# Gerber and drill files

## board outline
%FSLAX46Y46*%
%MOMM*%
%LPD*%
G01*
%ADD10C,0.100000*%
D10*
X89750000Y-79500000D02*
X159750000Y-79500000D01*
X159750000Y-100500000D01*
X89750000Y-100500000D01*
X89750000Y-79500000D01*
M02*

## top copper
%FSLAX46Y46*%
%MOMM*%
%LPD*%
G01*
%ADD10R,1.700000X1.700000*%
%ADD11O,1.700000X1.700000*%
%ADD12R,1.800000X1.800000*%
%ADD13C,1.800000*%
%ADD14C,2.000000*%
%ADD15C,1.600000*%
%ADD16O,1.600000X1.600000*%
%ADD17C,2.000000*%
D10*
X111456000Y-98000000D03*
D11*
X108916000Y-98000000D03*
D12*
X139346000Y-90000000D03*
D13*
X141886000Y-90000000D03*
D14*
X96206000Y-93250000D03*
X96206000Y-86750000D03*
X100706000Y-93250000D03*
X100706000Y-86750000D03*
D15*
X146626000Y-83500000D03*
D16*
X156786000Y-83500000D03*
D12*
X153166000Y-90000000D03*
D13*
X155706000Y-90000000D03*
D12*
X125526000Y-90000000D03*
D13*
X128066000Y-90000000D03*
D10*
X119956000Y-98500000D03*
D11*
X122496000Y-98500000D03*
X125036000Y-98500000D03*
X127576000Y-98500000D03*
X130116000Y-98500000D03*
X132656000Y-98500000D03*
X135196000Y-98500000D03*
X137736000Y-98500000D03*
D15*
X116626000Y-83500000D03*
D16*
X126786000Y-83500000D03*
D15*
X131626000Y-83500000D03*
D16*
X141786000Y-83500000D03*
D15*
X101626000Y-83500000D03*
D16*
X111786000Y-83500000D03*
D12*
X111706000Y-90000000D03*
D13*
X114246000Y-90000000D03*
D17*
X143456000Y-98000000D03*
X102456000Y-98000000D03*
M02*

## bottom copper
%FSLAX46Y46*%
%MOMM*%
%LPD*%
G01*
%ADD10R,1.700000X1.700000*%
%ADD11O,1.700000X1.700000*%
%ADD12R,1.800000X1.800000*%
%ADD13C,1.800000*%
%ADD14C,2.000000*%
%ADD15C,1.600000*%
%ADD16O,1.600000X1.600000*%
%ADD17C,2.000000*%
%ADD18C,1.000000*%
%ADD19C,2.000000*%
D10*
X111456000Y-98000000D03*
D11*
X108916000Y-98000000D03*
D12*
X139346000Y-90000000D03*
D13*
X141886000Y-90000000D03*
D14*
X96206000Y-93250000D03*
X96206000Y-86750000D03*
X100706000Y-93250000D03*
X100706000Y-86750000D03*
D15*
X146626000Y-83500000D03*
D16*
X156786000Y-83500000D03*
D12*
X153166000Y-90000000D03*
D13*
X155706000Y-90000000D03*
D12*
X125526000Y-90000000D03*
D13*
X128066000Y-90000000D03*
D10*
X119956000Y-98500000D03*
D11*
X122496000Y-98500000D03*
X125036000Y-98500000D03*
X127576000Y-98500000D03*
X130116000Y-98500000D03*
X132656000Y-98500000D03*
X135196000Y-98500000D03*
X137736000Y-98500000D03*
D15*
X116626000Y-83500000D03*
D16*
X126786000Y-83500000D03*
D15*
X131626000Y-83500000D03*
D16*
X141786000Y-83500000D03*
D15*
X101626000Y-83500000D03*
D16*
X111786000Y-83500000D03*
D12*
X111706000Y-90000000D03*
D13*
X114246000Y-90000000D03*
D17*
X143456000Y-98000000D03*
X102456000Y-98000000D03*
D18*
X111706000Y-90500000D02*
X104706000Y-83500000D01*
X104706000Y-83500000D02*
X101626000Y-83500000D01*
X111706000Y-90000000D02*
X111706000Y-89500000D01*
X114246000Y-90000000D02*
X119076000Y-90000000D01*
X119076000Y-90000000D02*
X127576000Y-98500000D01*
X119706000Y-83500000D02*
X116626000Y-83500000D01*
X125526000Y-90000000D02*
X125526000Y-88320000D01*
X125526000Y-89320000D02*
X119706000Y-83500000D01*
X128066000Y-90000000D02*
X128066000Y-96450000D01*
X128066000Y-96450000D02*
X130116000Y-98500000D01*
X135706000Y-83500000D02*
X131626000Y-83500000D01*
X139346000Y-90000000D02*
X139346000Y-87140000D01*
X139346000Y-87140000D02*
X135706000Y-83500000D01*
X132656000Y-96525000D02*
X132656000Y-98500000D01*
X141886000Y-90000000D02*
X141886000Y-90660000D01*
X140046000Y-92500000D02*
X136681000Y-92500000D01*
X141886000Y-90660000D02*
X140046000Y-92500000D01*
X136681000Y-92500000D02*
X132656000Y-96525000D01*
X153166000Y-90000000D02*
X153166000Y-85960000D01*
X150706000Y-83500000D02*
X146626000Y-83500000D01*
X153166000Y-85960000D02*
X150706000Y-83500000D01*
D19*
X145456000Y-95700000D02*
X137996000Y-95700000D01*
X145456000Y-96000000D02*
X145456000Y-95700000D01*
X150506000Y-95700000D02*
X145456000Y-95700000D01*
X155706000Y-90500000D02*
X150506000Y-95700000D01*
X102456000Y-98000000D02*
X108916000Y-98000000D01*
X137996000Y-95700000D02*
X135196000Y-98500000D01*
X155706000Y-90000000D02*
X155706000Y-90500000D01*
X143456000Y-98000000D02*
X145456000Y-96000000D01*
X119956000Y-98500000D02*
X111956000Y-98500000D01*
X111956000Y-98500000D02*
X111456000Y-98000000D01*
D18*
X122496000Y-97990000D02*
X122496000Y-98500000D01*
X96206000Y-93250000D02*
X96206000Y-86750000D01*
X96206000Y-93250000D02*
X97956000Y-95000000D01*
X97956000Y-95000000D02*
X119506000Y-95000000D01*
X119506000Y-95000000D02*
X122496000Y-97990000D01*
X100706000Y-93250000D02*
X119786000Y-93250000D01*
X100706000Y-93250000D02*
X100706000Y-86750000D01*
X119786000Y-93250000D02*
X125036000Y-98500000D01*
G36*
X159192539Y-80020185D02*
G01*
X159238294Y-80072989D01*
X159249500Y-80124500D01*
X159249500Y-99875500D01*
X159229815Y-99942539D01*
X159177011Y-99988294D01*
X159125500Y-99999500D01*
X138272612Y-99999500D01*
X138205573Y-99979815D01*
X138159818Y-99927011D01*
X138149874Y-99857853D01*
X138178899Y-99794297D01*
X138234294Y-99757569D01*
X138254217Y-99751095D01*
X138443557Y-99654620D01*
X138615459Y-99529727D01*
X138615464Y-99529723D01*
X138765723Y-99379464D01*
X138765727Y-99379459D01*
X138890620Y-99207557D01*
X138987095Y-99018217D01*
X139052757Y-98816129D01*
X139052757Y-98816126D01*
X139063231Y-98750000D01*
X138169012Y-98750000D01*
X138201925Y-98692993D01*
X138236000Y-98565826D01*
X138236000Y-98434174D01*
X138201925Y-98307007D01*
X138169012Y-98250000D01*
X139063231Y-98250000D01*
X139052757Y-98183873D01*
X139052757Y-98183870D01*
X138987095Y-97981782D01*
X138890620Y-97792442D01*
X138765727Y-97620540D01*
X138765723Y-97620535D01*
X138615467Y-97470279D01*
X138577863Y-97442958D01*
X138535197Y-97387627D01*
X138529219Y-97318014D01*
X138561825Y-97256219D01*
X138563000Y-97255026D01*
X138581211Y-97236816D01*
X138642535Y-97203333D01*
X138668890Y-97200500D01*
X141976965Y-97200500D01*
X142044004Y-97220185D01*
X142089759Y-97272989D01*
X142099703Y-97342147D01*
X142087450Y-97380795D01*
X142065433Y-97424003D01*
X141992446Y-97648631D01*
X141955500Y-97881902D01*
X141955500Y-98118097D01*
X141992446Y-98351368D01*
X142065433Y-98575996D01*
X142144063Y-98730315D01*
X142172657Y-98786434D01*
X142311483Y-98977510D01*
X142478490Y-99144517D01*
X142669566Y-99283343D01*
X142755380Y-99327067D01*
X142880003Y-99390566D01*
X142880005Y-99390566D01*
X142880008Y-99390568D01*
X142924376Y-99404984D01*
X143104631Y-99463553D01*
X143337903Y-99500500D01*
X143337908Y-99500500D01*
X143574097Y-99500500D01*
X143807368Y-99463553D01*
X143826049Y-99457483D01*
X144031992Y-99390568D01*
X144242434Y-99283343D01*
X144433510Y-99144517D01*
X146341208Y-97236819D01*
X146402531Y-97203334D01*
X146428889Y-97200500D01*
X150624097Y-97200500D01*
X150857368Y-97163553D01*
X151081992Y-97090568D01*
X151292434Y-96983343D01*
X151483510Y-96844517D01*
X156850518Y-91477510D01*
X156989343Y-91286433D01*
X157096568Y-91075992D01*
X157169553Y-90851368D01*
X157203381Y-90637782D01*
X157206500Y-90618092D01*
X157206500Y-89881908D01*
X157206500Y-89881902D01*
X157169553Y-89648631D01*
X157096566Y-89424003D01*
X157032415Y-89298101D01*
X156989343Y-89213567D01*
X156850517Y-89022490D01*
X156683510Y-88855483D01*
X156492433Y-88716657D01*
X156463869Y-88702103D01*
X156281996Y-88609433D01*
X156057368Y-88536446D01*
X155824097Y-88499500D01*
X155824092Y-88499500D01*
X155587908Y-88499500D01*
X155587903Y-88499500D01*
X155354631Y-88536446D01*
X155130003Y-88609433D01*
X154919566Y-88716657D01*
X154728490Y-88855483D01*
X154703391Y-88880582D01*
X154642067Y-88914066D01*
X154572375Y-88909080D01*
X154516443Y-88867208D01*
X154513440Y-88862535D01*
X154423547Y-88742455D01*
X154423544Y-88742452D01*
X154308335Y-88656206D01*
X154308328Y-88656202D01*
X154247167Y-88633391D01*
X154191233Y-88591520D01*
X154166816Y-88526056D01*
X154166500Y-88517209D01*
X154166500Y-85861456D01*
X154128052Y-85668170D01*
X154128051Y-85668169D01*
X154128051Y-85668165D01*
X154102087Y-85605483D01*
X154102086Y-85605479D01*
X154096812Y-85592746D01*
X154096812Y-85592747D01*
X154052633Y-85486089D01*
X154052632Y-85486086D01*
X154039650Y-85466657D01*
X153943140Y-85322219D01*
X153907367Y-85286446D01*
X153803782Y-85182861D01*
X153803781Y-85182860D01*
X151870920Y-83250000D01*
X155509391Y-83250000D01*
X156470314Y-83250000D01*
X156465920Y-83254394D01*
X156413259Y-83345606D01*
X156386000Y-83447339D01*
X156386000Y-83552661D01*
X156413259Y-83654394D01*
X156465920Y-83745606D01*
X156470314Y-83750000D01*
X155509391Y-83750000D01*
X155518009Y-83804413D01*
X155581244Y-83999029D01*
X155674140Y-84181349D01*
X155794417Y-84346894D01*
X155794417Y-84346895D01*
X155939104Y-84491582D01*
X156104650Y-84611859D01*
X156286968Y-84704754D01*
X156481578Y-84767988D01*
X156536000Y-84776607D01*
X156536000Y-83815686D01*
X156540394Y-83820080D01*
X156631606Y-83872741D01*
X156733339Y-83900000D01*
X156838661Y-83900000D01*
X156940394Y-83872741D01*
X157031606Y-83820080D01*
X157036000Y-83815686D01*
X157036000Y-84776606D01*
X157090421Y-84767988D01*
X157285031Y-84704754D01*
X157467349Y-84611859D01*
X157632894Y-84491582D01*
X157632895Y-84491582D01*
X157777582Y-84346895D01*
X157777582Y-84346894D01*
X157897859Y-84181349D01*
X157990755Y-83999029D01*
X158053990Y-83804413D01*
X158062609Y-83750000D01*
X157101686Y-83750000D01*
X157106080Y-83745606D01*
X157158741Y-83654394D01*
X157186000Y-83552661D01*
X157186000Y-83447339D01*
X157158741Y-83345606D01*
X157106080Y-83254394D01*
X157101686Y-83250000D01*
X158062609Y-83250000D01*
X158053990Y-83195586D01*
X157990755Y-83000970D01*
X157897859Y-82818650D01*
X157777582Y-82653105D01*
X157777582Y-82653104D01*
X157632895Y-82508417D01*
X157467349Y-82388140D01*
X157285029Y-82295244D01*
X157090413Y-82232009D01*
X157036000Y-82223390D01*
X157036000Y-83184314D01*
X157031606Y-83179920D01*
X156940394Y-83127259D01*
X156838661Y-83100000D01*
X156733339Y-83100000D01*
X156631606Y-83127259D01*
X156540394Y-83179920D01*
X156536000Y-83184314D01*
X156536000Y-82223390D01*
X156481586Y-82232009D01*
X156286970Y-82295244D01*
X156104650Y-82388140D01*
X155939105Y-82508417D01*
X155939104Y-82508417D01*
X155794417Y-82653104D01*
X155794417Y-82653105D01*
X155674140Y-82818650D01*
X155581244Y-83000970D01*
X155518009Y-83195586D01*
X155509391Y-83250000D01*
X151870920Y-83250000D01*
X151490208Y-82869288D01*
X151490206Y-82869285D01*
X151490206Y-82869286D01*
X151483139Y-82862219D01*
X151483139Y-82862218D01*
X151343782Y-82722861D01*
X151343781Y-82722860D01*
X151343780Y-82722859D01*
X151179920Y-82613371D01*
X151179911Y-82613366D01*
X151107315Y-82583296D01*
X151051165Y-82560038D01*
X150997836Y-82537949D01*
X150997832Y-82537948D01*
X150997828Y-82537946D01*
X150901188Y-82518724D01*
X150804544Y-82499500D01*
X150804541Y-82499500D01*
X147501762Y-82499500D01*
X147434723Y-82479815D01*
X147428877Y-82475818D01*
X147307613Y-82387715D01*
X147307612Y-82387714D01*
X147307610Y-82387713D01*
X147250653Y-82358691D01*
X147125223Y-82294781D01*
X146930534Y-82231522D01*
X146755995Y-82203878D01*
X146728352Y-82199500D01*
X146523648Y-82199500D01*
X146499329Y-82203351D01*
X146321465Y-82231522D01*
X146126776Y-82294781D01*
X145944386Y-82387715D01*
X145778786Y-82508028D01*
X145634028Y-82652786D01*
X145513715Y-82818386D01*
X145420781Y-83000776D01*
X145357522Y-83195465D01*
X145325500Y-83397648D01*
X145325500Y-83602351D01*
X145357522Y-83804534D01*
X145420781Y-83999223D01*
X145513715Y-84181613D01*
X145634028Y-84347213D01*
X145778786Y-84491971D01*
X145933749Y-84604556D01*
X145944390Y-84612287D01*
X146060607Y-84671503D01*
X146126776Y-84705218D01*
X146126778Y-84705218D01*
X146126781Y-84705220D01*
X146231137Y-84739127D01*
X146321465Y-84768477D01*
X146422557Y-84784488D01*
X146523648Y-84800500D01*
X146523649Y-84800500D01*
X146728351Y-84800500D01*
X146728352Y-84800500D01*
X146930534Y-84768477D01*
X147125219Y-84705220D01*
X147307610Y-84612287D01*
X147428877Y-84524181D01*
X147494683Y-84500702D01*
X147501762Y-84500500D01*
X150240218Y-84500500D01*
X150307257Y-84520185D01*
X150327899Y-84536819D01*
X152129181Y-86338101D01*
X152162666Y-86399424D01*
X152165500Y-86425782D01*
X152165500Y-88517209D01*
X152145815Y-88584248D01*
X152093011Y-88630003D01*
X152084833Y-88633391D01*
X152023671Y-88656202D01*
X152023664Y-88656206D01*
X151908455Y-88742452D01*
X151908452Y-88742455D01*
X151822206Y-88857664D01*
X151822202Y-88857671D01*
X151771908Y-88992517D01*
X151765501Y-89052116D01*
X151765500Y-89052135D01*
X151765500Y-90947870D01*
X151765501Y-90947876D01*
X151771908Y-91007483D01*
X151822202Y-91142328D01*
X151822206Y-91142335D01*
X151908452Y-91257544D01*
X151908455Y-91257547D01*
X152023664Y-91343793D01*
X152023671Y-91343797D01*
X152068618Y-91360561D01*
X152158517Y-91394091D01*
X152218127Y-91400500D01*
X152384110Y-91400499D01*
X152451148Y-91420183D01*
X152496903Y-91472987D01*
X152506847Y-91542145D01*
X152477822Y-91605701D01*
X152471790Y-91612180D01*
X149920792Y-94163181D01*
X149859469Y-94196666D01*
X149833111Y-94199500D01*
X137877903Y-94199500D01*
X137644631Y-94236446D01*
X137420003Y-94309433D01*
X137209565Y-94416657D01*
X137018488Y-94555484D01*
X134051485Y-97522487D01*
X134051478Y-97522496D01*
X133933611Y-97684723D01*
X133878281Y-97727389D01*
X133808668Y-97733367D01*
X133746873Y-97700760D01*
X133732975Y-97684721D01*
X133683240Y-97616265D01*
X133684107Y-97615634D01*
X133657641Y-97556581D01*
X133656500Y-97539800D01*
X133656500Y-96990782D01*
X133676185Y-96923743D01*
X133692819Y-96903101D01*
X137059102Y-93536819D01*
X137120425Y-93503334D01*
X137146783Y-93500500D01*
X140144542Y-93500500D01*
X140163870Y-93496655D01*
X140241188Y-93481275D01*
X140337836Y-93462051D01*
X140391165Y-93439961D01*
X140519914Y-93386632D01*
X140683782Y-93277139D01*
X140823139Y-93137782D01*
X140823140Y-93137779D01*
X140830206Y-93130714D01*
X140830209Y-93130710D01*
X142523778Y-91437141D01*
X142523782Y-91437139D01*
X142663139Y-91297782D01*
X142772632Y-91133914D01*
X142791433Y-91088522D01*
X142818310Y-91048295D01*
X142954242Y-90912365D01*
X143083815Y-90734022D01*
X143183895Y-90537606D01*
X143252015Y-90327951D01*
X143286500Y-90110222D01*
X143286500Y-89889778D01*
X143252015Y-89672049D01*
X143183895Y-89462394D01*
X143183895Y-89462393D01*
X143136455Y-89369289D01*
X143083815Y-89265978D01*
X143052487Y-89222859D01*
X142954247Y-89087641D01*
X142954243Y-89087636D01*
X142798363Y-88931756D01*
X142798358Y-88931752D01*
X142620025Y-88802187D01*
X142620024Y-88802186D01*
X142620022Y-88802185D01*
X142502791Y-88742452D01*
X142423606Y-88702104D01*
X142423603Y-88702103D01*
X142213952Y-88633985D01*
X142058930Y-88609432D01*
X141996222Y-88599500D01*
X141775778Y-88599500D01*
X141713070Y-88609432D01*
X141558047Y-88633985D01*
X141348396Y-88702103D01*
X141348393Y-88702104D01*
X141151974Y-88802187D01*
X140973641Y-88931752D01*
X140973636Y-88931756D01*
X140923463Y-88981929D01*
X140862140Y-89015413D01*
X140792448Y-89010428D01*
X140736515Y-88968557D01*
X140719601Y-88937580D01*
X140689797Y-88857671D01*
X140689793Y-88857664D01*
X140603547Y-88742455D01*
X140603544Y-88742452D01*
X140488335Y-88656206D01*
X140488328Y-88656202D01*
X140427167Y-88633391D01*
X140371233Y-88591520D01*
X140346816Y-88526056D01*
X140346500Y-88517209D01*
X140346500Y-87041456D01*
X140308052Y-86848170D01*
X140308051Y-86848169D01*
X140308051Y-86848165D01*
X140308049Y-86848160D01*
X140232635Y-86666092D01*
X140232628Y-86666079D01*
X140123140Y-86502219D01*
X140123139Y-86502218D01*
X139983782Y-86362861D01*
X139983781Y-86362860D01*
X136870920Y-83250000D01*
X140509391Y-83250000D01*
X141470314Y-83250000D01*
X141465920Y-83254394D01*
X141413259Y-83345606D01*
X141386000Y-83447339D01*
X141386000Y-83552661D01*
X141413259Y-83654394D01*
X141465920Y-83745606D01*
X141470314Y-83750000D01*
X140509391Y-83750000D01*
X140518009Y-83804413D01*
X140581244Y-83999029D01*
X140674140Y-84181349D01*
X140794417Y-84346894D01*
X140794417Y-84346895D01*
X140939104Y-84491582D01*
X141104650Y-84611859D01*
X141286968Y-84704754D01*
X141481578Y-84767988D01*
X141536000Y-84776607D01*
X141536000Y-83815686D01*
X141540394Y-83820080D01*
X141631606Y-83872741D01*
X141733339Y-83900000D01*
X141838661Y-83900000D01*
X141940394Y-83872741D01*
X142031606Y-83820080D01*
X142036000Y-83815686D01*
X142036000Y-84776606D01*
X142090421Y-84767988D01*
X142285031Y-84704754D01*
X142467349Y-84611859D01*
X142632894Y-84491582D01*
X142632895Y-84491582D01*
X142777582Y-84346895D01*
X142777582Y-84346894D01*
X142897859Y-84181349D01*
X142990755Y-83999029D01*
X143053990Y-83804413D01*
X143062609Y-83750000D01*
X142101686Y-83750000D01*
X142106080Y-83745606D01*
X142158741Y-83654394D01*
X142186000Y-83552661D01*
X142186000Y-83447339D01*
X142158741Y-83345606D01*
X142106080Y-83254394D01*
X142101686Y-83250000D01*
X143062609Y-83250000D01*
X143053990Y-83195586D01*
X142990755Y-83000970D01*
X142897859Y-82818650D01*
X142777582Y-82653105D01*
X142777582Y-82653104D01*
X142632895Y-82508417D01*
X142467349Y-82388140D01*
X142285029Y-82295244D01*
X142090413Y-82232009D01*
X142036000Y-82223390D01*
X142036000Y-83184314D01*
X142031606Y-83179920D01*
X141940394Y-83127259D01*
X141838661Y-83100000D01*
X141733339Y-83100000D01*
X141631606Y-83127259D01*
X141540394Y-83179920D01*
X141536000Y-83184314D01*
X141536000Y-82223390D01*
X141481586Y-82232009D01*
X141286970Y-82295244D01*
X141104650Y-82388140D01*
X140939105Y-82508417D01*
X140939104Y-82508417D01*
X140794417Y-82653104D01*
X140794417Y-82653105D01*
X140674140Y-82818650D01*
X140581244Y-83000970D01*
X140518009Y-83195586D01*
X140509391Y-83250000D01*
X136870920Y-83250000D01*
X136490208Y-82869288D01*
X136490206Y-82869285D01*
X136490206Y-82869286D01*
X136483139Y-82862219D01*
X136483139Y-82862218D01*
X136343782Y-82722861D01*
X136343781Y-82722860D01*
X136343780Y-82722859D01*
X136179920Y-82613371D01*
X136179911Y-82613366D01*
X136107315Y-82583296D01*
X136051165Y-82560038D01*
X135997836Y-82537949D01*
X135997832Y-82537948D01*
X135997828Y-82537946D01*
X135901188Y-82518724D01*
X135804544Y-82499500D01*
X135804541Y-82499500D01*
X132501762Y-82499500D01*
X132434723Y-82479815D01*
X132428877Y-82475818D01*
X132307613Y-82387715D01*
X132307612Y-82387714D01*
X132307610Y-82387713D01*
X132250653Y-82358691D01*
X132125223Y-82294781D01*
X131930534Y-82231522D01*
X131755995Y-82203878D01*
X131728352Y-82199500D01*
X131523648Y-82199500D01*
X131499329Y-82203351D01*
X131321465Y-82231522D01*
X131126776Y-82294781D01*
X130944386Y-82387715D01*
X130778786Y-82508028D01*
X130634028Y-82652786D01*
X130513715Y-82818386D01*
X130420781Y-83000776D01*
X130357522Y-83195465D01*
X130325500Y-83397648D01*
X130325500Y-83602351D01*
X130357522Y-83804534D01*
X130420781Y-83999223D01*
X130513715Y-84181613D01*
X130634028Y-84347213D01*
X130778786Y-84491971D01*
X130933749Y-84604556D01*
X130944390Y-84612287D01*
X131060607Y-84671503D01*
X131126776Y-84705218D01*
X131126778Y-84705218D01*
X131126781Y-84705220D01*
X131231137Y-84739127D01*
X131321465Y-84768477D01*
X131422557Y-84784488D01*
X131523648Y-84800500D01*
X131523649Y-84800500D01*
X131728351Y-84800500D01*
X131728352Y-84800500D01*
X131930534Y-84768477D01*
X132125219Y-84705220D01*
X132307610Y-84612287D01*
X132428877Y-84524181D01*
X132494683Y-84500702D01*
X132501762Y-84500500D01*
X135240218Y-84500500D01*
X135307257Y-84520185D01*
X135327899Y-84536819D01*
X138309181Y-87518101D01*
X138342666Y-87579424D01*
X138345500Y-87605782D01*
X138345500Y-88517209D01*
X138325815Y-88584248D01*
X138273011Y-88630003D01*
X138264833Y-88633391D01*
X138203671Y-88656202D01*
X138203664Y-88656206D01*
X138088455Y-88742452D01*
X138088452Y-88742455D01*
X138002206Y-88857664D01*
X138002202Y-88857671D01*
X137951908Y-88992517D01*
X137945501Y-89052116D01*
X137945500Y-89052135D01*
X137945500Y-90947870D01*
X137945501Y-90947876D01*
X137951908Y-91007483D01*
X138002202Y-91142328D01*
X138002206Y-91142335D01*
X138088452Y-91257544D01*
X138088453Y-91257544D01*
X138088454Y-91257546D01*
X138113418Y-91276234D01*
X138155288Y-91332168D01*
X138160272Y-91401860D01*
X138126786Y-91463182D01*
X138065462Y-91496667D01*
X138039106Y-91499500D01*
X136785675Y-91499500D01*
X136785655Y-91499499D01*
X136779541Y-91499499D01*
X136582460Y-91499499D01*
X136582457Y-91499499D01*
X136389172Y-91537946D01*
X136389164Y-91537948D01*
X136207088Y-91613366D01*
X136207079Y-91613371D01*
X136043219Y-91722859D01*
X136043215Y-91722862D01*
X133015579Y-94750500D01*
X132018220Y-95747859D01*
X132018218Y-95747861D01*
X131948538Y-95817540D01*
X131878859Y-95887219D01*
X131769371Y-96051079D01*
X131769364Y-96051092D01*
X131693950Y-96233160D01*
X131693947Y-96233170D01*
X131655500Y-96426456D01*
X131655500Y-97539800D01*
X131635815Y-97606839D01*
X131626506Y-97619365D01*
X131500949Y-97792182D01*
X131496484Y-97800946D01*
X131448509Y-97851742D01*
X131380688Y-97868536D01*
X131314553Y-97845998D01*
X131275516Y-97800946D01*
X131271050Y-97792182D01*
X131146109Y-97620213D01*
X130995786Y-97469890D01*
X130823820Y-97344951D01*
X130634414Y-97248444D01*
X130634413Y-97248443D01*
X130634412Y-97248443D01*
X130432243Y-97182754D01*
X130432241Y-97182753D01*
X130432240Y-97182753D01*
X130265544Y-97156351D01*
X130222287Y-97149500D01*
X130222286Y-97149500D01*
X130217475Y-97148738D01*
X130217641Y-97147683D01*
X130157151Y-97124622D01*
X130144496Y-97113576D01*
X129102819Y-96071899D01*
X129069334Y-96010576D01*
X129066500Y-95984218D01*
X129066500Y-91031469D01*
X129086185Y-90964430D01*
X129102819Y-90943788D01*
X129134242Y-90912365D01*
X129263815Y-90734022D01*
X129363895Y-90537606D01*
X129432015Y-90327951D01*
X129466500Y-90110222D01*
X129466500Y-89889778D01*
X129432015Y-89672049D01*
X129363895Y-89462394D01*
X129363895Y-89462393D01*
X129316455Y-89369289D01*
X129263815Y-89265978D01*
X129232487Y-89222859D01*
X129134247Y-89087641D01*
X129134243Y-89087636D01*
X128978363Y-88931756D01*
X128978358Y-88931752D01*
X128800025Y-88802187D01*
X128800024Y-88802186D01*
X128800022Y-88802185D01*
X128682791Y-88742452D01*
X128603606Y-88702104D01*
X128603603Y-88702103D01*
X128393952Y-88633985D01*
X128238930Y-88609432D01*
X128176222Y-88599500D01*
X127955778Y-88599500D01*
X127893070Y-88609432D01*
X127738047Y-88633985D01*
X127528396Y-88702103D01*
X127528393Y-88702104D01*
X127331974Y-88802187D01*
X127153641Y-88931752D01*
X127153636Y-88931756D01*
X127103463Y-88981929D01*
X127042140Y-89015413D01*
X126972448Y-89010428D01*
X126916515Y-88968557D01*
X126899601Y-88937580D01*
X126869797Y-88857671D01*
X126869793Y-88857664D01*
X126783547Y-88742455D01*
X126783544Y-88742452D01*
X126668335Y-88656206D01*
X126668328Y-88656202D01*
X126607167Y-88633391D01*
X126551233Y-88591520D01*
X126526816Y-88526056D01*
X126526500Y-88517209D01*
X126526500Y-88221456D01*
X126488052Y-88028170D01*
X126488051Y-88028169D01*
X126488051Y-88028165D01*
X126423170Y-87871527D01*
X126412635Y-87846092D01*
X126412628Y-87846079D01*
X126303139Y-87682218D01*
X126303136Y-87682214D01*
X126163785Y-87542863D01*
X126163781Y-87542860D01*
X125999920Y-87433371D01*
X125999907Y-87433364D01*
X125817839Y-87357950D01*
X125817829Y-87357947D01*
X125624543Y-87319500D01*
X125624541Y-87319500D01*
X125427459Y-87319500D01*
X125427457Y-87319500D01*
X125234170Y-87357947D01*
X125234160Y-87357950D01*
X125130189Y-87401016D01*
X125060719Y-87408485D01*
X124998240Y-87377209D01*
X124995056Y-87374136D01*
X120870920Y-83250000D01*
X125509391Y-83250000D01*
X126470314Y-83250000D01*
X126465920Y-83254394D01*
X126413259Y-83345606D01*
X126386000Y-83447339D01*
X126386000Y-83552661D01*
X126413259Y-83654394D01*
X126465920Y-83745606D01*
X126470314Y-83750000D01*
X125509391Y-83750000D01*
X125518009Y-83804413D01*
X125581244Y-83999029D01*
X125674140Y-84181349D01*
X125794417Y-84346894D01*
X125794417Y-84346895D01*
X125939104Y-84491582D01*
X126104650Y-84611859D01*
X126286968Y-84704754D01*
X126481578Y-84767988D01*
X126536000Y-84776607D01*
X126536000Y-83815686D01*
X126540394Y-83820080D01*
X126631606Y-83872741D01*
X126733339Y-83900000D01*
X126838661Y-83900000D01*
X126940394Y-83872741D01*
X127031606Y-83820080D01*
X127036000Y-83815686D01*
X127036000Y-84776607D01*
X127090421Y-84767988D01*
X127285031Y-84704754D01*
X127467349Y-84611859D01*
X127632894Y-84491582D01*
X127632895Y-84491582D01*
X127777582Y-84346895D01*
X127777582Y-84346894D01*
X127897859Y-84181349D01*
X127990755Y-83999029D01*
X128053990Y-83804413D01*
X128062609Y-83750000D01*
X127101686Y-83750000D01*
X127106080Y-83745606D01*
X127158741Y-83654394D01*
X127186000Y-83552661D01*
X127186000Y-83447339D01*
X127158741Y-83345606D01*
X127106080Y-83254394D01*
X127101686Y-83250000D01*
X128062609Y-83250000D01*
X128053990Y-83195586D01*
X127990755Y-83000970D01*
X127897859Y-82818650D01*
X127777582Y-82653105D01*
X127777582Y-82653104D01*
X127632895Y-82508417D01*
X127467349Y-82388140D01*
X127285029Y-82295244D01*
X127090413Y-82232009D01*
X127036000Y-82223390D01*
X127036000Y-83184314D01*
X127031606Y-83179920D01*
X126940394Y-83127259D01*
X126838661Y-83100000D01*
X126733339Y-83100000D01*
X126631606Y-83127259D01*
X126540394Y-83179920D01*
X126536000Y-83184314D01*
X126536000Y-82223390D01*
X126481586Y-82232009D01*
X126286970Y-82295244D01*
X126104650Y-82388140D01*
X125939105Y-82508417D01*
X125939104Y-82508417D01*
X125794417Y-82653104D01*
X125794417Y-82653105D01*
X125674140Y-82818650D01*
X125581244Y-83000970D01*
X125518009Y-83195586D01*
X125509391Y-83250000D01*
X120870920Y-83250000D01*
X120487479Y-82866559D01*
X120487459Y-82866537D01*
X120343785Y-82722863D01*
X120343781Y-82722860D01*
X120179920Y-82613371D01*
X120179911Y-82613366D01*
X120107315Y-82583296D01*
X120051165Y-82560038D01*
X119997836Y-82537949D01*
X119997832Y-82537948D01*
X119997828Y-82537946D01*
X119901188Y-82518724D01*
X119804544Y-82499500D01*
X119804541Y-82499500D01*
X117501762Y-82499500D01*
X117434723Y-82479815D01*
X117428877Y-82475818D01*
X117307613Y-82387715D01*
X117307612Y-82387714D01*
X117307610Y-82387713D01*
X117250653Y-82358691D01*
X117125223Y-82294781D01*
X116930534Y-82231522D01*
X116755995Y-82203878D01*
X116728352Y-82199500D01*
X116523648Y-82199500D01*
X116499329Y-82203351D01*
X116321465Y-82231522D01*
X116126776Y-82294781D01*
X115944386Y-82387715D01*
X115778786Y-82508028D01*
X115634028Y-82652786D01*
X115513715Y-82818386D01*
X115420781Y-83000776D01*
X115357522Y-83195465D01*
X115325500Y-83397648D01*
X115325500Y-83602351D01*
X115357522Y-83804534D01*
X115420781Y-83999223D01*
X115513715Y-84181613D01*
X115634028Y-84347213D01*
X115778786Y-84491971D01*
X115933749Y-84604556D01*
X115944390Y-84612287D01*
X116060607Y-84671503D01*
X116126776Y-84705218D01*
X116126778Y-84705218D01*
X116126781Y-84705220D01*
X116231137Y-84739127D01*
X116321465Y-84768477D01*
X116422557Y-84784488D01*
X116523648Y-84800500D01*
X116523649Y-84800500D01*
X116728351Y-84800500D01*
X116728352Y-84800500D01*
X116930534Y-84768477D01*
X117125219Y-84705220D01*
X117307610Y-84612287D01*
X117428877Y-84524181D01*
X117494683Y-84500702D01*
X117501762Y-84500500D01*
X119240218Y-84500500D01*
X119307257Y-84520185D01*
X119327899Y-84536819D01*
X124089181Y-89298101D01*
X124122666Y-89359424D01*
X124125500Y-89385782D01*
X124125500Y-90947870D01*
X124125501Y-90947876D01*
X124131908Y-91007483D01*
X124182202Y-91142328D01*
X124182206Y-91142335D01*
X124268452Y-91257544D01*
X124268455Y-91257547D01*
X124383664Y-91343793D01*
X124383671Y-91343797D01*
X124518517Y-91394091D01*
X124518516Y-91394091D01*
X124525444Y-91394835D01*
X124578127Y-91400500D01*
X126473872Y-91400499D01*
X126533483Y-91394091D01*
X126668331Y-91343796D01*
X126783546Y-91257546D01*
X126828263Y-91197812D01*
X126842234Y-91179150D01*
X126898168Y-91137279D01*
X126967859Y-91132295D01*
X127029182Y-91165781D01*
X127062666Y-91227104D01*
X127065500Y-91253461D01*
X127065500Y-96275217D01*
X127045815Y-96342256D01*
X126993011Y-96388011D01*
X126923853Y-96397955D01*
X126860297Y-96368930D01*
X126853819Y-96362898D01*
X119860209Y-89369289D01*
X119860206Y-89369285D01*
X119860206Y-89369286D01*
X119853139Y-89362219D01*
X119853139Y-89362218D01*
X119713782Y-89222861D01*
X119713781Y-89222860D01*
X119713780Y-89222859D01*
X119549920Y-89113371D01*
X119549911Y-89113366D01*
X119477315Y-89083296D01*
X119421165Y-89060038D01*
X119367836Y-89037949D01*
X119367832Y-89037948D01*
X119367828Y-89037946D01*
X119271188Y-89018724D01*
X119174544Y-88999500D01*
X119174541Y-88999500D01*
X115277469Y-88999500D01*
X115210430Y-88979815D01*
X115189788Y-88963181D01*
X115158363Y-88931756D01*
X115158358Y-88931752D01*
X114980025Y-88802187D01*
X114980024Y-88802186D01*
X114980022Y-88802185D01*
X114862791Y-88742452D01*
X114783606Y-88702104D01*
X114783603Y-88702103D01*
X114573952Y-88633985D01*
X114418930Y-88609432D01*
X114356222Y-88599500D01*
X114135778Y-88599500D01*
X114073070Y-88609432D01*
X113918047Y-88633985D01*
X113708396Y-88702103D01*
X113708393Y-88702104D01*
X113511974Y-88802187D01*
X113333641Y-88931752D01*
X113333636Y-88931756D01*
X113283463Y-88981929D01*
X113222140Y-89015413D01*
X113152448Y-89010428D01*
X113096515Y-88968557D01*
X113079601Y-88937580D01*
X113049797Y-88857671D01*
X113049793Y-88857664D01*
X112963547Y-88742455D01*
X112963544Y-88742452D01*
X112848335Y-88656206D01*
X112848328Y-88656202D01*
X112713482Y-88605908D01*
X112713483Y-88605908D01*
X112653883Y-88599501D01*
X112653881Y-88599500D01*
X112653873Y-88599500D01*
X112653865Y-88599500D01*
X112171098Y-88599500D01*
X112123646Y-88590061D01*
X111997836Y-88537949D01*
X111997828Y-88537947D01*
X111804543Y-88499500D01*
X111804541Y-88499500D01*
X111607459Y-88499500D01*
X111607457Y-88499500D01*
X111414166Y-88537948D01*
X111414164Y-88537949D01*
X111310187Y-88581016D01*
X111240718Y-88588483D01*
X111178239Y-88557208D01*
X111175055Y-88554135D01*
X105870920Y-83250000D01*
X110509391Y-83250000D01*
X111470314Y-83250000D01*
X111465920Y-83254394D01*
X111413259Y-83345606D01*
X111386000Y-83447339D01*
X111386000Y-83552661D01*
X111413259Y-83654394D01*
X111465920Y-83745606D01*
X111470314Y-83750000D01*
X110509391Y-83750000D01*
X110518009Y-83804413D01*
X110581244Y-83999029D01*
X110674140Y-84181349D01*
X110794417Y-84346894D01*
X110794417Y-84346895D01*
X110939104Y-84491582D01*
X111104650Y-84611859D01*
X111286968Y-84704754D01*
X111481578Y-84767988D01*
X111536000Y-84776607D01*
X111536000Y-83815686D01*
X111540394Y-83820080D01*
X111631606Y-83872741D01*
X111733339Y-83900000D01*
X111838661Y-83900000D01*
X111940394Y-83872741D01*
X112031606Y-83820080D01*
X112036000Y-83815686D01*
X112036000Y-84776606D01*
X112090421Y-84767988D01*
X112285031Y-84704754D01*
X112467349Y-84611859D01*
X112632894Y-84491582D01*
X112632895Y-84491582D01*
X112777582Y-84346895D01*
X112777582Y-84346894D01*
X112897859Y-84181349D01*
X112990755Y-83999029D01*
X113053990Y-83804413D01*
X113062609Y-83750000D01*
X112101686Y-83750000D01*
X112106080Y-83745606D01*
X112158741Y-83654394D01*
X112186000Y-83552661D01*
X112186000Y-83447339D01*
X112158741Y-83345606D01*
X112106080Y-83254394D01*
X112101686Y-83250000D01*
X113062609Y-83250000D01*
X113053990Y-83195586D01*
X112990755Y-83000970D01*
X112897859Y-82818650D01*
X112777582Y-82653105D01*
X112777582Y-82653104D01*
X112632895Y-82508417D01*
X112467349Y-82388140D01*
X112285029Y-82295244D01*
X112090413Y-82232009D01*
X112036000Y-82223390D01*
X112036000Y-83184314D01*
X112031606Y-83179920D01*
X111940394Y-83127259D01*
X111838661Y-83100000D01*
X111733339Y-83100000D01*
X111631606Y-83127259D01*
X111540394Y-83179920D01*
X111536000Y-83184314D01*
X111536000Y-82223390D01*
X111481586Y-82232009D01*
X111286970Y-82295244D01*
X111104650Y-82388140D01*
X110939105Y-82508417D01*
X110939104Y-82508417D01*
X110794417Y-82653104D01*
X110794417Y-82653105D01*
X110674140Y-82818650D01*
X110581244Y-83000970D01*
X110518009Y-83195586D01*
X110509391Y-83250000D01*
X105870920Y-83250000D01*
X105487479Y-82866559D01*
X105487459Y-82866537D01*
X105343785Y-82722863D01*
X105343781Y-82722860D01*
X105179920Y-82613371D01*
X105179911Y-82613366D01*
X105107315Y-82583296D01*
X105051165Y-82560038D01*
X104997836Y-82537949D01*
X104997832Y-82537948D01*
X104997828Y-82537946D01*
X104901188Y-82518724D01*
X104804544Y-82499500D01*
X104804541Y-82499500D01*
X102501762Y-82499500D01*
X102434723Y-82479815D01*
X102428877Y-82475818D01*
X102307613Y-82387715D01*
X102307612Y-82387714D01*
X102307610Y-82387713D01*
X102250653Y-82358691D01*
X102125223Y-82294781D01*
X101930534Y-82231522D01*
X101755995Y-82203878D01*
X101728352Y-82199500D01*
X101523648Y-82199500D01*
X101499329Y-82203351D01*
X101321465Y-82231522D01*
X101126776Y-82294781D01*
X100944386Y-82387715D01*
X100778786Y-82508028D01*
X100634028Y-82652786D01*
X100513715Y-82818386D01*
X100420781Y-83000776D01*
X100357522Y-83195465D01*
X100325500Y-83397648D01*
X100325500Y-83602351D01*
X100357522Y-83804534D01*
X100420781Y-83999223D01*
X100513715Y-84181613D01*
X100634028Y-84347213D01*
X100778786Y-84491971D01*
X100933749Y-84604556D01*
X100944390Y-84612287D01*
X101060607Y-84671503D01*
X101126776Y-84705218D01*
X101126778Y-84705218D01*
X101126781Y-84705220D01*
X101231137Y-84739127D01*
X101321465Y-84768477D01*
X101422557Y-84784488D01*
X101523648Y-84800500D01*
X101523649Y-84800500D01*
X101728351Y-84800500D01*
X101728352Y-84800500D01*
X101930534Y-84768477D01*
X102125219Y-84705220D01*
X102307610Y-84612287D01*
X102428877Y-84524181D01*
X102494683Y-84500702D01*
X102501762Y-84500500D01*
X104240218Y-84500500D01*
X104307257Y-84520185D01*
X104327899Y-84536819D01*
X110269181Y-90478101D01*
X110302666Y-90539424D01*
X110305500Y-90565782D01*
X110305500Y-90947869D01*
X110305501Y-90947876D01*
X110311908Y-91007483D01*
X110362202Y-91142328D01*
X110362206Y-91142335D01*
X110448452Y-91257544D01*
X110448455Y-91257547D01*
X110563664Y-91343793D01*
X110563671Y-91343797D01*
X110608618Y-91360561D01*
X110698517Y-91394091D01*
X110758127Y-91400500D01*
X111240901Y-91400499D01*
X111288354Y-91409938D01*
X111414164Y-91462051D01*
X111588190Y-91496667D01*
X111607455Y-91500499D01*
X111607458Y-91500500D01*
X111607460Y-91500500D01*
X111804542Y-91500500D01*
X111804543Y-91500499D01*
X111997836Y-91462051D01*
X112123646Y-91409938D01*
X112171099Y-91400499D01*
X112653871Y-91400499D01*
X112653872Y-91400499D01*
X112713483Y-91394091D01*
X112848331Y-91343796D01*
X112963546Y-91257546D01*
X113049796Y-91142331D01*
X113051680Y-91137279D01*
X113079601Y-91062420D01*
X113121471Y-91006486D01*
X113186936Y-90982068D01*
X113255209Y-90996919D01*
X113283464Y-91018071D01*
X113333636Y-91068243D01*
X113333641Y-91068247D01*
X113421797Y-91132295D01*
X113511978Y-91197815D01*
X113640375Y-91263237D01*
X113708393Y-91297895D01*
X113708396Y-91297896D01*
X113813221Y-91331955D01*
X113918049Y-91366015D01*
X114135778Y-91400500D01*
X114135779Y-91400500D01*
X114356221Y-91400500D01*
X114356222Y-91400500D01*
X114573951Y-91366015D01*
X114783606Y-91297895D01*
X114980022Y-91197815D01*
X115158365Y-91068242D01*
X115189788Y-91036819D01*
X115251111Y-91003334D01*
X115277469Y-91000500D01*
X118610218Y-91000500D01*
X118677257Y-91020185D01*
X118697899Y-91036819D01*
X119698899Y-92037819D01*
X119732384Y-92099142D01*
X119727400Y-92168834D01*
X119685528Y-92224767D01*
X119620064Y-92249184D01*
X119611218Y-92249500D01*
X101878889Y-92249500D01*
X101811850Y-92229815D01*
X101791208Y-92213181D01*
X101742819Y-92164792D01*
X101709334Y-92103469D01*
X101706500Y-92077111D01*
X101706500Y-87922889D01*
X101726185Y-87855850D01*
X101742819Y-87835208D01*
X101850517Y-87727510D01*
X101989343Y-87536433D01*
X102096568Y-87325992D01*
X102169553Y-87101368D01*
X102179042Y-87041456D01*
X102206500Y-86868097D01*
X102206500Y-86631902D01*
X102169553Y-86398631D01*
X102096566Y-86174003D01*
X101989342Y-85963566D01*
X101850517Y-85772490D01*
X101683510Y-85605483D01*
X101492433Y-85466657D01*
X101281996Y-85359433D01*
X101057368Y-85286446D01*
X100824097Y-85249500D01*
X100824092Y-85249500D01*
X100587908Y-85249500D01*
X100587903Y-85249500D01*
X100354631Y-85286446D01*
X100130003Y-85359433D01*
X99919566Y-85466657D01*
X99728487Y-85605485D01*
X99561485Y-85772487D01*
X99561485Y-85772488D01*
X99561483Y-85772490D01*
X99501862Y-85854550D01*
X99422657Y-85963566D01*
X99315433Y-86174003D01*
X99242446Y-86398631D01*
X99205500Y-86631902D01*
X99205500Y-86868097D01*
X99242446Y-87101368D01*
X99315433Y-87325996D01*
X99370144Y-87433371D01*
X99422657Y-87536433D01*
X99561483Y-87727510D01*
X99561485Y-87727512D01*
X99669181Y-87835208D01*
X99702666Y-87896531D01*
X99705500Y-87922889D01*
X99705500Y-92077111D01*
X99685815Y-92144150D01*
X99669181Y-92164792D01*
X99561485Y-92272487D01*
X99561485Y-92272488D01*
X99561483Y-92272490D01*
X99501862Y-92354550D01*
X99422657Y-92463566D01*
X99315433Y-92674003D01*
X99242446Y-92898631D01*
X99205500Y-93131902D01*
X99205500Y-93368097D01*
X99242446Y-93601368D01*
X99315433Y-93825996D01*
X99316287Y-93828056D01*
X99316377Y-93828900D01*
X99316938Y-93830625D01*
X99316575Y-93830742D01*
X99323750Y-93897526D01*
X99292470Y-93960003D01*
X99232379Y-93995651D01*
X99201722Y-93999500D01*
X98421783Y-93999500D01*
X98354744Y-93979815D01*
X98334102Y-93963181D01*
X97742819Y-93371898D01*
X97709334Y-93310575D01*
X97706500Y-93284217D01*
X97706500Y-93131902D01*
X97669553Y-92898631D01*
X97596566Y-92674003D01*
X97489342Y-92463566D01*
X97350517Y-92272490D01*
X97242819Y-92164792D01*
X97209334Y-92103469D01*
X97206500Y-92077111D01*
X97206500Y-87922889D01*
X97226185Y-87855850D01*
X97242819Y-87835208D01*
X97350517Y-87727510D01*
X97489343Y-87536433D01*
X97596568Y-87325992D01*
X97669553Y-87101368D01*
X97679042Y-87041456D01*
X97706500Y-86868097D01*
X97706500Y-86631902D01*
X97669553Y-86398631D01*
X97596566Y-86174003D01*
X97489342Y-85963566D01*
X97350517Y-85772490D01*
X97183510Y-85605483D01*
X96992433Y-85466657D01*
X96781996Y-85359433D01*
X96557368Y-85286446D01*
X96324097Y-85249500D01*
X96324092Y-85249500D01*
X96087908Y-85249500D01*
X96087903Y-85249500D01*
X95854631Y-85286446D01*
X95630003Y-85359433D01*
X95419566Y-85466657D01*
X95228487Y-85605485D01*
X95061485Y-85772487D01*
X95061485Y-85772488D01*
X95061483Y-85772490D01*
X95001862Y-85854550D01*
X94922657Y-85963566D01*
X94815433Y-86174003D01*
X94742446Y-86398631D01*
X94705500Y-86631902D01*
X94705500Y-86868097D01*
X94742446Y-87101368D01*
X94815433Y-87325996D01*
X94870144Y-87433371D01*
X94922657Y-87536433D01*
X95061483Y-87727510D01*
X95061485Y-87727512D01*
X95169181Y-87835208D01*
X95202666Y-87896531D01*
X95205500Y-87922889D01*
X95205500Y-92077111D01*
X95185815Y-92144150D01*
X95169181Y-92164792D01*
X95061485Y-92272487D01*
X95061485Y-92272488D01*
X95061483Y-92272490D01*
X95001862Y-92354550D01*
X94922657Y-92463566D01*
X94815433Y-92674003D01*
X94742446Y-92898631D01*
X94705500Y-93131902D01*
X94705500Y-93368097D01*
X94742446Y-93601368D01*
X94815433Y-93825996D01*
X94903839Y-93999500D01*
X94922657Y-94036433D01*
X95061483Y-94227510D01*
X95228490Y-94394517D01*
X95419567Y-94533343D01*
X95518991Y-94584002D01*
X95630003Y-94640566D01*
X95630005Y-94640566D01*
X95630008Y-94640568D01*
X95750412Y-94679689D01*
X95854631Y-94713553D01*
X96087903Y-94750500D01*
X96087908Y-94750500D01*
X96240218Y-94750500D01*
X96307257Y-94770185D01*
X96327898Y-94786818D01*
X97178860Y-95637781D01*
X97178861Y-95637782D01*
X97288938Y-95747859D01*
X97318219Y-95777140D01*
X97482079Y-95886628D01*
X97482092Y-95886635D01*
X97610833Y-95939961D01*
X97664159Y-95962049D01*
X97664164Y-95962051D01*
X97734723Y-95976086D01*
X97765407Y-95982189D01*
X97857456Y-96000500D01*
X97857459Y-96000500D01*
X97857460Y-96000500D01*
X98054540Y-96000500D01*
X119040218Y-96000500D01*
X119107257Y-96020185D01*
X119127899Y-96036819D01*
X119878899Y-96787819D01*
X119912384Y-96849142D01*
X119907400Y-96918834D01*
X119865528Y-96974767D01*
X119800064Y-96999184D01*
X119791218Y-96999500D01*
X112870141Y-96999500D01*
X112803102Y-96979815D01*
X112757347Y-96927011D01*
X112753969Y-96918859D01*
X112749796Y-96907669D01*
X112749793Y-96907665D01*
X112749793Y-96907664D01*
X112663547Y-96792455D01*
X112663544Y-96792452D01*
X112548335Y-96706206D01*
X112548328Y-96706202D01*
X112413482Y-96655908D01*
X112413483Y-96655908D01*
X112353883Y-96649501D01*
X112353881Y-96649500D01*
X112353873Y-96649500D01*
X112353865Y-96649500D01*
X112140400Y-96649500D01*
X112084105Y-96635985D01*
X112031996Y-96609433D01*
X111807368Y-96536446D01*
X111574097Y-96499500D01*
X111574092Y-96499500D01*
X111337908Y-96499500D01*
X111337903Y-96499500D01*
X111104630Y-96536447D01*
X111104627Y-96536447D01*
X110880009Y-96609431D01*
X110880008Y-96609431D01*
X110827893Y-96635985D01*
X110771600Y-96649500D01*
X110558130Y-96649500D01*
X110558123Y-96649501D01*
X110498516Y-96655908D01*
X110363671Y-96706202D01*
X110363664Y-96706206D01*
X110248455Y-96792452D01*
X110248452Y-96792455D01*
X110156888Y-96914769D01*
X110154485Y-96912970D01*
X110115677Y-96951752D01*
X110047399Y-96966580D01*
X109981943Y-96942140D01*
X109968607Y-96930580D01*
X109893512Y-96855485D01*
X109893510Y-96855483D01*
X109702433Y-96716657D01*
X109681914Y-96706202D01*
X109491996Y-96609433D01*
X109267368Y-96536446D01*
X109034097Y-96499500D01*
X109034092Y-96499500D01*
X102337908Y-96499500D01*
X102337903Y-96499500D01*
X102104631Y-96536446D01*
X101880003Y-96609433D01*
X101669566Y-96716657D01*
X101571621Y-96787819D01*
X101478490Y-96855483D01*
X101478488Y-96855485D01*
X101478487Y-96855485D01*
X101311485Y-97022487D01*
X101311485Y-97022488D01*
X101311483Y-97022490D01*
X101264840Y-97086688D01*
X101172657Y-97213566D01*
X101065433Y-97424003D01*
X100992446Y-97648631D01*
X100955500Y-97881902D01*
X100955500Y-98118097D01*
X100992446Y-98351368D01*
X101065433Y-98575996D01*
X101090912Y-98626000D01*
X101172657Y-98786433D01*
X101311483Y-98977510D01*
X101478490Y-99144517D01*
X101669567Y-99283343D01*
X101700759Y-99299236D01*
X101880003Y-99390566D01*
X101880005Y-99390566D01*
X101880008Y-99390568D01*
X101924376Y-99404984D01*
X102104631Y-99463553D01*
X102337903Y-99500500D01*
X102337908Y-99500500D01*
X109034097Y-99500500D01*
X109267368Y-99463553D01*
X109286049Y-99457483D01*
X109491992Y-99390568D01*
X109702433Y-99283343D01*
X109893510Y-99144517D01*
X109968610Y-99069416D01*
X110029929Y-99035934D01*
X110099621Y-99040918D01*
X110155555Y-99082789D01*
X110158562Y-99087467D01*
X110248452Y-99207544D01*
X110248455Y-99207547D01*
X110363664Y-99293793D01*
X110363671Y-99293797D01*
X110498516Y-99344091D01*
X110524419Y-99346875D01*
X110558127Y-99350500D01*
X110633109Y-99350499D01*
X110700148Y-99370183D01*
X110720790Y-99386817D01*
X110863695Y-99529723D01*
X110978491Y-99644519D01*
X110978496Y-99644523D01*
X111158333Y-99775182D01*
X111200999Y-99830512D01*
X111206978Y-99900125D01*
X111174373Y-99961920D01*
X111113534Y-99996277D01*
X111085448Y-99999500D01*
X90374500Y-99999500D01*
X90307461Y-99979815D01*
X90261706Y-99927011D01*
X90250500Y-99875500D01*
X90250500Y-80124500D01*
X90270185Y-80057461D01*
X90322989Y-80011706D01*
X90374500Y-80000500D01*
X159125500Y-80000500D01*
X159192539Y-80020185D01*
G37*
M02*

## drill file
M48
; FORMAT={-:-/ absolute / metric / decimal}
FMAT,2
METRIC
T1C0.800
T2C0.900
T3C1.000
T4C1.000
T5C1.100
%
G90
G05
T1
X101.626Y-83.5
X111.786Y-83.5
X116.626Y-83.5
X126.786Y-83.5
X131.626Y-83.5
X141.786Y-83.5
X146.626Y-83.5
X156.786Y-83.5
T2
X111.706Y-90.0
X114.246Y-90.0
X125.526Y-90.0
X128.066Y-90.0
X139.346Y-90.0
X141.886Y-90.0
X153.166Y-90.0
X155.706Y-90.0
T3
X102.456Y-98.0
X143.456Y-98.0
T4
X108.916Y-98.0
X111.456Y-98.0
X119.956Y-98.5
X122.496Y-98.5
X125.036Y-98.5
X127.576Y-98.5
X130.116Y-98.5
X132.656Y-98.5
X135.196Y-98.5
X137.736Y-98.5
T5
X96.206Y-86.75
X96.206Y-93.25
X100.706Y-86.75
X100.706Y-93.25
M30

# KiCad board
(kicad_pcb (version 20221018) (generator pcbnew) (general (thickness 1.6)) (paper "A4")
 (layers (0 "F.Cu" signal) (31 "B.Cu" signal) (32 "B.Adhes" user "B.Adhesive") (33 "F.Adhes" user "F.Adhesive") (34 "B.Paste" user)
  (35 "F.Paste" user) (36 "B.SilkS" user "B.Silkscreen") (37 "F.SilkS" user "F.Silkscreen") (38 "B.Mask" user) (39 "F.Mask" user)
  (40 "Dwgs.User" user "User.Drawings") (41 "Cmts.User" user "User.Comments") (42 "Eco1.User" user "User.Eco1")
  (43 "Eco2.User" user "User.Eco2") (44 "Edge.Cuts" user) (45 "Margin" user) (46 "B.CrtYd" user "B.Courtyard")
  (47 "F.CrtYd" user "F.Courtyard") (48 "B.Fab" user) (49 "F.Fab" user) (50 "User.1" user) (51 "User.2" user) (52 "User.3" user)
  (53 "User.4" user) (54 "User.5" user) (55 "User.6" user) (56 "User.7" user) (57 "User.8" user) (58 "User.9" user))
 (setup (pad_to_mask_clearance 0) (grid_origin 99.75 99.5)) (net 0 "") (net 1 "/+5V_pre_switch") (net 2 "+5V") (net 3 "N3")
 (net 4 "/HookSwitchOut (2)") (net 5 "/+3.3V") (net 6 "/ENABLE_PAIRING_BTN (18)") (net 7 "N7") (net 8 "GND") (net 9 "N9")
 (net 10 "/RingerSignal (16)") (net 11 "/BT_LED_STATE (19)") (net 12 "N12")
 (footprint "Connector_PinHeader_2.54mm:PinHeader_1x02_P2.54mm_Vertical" (layer "F.Cu") (at 111.456 98 -90)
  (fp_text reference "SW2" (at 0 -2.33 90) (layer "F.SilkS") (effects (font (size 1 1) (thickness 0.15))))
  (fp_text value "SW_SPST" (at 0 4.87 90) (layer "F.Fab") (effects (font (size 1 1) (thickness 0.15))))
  (pad "1" thru_hole rect (at 0 0 270) (size 1.7 1.7) (drill 1) (layers "*.Cu" "*.Mask") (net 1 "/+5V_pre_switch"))
  (pad "2" thru_hole oval (at 0 2.54 270) (size 1.7 1.7) (drill 1) (layers "*.Cu" "*.Mask") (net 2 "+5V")))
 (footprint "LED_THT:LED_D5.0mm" (layer "F.Cu") (at 139.346 90)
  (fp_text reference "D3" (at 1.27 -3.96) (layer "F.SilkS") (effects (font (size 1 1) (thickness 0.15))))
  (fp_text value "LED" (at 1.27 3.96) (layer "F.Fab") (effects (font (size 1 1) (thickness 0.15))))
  (pad "1" thru_hole rect (at 0 0) (size 1.8 1.8) (drill 0.9) (layers "*.Cu" "*.Mask") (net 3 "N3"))
  (pad "2" thru_hole circle (at 2.54 0) (size 1.8 1.8) (drill 0.9) (layers "*.Cu" "*.Mask") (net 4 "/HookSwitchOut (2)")))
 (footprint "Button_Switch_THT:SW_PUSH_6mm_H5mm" (layer "F.Cu") (at 96.206 93.25 90)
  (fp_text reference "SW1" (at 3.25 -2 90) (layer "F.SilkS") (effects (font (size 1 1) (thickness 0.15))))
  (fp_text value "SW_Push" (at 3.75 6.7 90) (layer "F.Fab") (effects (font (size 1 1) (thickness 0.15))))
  (pad "1" thru_hole circle (at 0 0 180) (size 2 2) (drill 1.1) (layers "*.Cu" "*.Mask") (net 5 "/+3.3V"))
  (pad "1" thru_hole circle (at 6.5 0 180) (size 2 2) (drill 1.1) (layers "*.Cu" "*.Mask") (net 5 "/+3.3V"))
  (pad "2" thru_hole circle (at 0 4.5 180) (size 2 2) (drill 1.1) (layers "*.Cu" "*.Mask") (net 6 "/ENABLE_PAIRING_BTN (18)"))
  (pad "2" thru_hole circle (at 6.5 4.5 180) (size 2 2) (drill 1.1) (layers "*.Cu" "*.Mask") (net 6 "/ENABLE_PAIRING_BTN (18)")))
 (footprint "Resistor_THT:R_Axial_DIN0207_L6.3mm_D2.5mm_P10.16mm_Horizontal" (layer "F.Cu") (at 146.626 83.5)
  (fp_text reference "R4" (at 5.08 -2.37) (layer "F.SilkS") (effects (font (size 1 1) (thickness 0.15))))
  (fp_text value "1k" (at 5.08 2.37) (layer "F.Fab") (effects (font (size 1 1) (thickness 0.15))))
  (pad "1" thru_hole circle (at 0 0) (size 1.6 1.6) (drill 0.8) (layers "*.Cu" "*.Mask") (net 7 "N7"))
  (pad "2" thru_hole oval (at 10.16 0) (size 1.6 1.6) (drill 0.8) (layers "*.Cu" "*.Mask") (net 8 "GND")))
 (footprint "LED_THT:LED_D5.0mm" (layer "F.Cu") (at 153.166 90)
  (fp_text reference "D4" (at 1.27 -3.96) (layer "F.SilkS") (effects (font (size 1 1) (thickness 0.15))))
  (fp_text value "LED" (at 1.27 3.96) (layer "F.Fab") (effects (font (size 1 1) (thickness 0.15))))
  (pad "1" thru_hole rect (at 0 0) (size 1.8 1.8) (drill 0.9) (layers "*.Cu" "*.Mask") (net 7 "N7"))
  (pad "2" thru_hole circle (at 2.54 0) (size 1.8 1.8) (drill 0.9) (layers "*.Cu" "*.Mask") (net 2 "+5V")))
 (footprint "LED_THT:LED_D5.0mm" (layer "F.Cu") (at 125.526 90)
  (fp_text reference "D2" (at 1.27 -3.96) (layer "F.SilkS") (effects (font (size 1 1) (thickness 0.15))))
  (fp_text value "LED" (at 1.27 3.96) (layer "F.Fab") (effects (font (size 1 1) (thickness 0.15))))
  (pad "1" thru_hole rect (at 0 0) (size 1.8 1.8) (drill 0.9) (layers "*.Cu" "*.Mask") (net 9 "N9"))
  (pad "2" thru_hole circle (at 2.54 0) (size 1.8 1.8) (drill 0.9) (layers "*.Cu" "*.Mask") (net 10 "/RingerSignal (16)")))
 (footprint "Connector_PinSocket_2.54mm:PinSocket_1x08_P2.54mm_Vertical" (layer "F.Cu") (at 119.956 98.5 90)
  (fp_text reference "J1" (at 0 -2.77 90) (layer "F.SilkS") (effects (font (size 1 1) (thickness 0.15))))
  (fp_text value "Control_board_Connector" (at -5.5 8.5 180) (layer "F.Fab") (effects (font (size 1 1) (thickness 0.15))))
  (pad "1" thru_hole rect (at 0 0 90) (size 1.7 1.7) (drill 1) (layers "*.Cu" "*.Mask") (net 1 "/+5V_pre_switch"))
  (pad "2" thru_hole oval (at 0 2.54 90) (size 1.7 1.7) (drill 1) (layers "*.Cu" "*.Mask") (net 5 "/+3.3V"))
  (pad "3" thru_hole oval (at 0 5.08 90) (size 1.7 1.7) (drill 1) (layers "*.Cu" "*.Mask") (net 6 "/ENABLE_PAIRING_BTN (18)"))
  (pad "4" thru_hole oval (at 0 7.62 90) (size 1.7 1.7) (drill 1) (layers "*.Cu" "*.Mask") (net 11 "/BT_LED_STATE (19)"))
  (pad "5" thru_hole oval (at 0 10.16 90) (size 1.7 1.7) (drill 1) (layers "*.Cu" "*.Mask") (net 10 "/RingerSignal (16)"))
  (pad "6" thru_hole oval (at 0 12.7 90) (size 1.7 1.7) (drill 1) (layers "*.Cu" "*.Mask") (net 4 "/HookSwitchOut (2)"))
  (pad "7" thru_hole oval (at 0 15.24 90) (size 1.7 1.7) (drill 1) (layers "*.Cu" "*.Mask") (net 2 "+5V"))
  (pad "8" thru_hole oval (at 0 17.78 90) (size 1.7 1.7) (drill 1) (layers "*.Cu" "*.Mask") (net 8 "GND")))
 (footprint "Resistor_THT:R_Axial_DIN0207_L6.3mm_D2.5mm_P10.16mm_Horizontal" (layer "F.Cu") (at 116.626 83.5)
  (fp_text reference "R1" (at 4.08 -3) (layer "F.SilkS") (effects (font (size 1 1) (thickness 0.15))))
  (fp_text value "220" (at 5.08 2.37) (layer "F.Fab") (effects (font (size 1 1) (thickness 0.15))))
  (pad "1" thru_hole circle (at 0 0) (size 1.6 1.6) (drill 0.8) (layers "*.Cu" "*.Mask") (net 9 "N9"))
  (pad "2" thru_hole oval (at 10.16 0) (size 1.6 1.6) (drill 0.8) (layers "*.Cu" "*.Mask") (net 8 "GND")))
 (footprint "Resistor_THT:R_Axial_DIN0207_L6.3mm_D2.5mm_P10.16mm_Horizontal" (layer "F.Cu") (at 131.626 83.5)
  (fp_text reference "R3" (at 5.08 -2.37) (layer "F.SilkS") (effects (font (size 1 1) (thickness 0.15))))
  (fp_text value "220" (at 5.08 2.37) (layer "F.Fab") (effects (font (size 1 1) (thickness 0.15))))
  (pad "1" thru_hole circle (at 0 0) (size 1.6 1.6) (drill 0.8) (layers "*.Cu" "*.Mask") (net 3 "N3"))
  (pad "2" thru_hole oval (at 10.16 0) (size 1.6 1.6) (drill 0.8) (layers "*.Cu" "*.Mask") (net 8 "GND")))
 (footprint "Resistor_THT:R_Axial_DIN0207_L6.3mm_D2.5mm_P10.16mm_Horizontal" (layer "F.Cu") (at 101.626 83.5)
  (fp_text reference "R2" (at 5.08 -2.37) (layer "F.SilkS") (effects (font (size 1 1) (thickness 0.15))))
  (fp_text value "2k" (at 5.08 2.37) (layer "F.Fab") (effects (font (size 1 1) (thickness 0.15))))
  (pad "1" thru_hole circle (at 0 0) (size 1.6 1.6) (drill 0.8) (layers "*.Cu" "*.Mask") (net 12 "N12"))
  (pad "2" thru_hole oval (at 10.16 0) (size 1.6 1.6) (drill 0.8) (layers "*.Cu" "*.Mask") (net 8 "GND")))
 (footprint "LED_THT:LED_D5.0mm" (layer "F.Cu") (at 111.706 90)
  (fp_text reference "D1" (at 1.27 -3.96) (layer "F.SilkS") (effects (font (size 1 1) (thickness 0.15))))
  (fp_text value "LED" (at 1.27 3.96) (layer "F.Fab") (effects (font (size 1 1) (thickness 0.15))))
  (pad "1" thru_hole rect (at 0 0) (size 1.8 1.8) (drill 0.9) (layers "*.Cu" "*.Mask") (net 12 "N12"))
  (pad "2" thru_hole circle (at 2.54 0) (size 1.8 1.8) (drill 0.9) (layers "*.Cu" "*.Mask") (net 11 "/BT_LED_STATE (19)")))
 (gr_rect (start 89.75 79.5) (end 159.75 100.5) (stroke (width 0.1) (type default)) (fill none) (layer "Edge.Cuts"))
 (segment (start 111.706 90.5) (end 104.706 83.5) (width 1) (layer "B.Cu") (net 12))
 (segment (start 104.706 83.5) (end 101.626 83.5) (width 1) (layer "B.Cu") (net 12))
 (segment (start 111.706 90) (end 111.706 89.5) (width 1) (layer "B.Cu") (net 12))
 (segment (start 114.246 90) (end 119.076 90) (width 1) (layer "B.Cu") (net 11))
 (segment (start 119.076 90) (end 127.576 98.5) (width 1) (layer "B.Cu") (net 11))
 (segment (start 119.706 83.5) (end 116.626 83.5) (width 1) (layer "B.Cu") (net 9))
 (segment (start 125.526 90) (end 125.526 88.32) (width 1) (layer "B.Cu") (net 9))
 (segment (start 125.526 89.32) (end 119.706 83.5) (width 1) (layer "B.Cu") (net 9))
 (segment (start 128.066 90) (end 128.066 96.45) (width 1) (layer "B.Cu") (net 10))
 (segment (start 128.066 96.45) (end 130.116 98.5) (width 1) (layer "B.Cu") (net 10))
 (segment (start 135.706 83.5) (end 131.626 83.5) (width 1) (layer "B.Cu") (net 3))
 (segment (start 139.346 90) (end 139.346 87.14) (width 1) (layer "B.Cu") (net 3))
 (segment (start 139.346 87.14) (end 135.706 83.5) (width 1) (layer "B.Cu") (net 3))
 (segment (start 132.656 96.525) (end 132.656 98.5) (width 1) (layer "B.Cu") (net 4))
 (segment (start 141.886 90) (end 141.886 90.66) (width 1) (layer "B.Cu") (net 4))
 (segment (start 140.046 92.5) (end 136.681 92.5) (width 1) (layer "B.Cu") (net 4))
 (segment (start 141.886 90.66) (end 140.046 92.5) (width 1) (layer "B.Cu") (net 4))
 (segment (start 136.681 92.5) (end 132.656 96.525) (width 1) (layer "B.Cu") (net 4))
 (segment (start 153.166 90) (end 153.166 85.96) (width 1) (layer "B.Cu") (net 7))
 (segment (start 150.706 83.5) (end 146.626 83.5) (width 1) (layer "B.Cu") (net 7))
 (segment (start 153.166 85.96) (end 150.706 83.5) (width 1) (layer "B.Cu") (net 7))
 (via (at 143.456 98) (size 2) (drill 1) (layers "F.Cu" "B.Cu") (free) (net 2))
 (via (at 102.456 98) (size 2) (drill 1) (layers "F.Cu" "B.Cu") (free) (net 2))
 (segment (start 145.456 95.7) (end 137.996 95.7) (width 2) (layer "B.Cu") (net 2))
 (segment (start 145.456 96) (end 145.456 95.7) (width 2) (layer "B.Cu") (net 2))
 (segment (start 150.506 95.7) (end 145.456 95.7) (width 2) (layer "B.Cu") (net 2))
 (segment (start 155.706 90.5) (end 150.506 95.7) (width 2) (layer "B.Cu") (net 2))
 (segment (start 102.456 98) (end 108.916 98) (width 2) (layer "B.Cu") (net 2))
 (segment (start 137.996 95.7) (end 135.196 98.5) (width 2) (layer "B.Cu") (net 2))
 (segment (start 155.706 90) (end 155.706 90.5) (width 2) (layer "B.Cu") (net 2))
 (segment (start 143.456 98) (end 145.456 96) (width 2) (layer "B.Cu") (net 2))
 (segment (start 119.956 98.5) (end 111.956 98.5) (width 2) (layer "B.Cu") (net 1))
 (segment (start 111.956 98.5) (end 111.456 98) (width 2) (layer "B.Cu") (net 1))
 (segment (start 122.496 97.99) (end 122.496 98.5) (width 1) (layer "B.Cu") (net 5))
 (segment (start 96.206 93.25) (end 96.206 86.75) (width 1) (layer "B.Cu") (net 5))
 (segment (start 96.206 93.25) (end 97.956 95) (width 1) (layer "B.Cu") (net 5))
 (segment (start 97.956 95) (end 119.506 95) (width 1) (layer "B.Cu") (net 5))
 (segment (start 119.506 95) (end 122.496 97.99) (width 1) (layer "B.Cu") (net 5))
 (segment (start 100.706 93.25) (end 119.786 93.25) (width 1) (layer "B.Cu") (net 6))
 (segment (start 100.706 93.25) (end 100.706 86.75) (width 1) (layer "B.Cu") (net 6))
 (segment (start 119.786 93.25) (end 125.036 98.5) (width 1) (layer "B.Cu") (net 6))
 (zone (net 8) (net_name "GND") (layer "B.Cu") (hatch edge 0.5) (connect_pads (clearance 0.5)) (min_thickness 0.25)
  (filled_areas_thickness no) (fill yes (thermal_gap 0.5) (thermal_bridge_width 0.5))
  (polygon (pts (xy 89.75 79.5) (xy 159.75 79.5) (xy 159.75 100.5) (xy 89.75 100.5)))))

